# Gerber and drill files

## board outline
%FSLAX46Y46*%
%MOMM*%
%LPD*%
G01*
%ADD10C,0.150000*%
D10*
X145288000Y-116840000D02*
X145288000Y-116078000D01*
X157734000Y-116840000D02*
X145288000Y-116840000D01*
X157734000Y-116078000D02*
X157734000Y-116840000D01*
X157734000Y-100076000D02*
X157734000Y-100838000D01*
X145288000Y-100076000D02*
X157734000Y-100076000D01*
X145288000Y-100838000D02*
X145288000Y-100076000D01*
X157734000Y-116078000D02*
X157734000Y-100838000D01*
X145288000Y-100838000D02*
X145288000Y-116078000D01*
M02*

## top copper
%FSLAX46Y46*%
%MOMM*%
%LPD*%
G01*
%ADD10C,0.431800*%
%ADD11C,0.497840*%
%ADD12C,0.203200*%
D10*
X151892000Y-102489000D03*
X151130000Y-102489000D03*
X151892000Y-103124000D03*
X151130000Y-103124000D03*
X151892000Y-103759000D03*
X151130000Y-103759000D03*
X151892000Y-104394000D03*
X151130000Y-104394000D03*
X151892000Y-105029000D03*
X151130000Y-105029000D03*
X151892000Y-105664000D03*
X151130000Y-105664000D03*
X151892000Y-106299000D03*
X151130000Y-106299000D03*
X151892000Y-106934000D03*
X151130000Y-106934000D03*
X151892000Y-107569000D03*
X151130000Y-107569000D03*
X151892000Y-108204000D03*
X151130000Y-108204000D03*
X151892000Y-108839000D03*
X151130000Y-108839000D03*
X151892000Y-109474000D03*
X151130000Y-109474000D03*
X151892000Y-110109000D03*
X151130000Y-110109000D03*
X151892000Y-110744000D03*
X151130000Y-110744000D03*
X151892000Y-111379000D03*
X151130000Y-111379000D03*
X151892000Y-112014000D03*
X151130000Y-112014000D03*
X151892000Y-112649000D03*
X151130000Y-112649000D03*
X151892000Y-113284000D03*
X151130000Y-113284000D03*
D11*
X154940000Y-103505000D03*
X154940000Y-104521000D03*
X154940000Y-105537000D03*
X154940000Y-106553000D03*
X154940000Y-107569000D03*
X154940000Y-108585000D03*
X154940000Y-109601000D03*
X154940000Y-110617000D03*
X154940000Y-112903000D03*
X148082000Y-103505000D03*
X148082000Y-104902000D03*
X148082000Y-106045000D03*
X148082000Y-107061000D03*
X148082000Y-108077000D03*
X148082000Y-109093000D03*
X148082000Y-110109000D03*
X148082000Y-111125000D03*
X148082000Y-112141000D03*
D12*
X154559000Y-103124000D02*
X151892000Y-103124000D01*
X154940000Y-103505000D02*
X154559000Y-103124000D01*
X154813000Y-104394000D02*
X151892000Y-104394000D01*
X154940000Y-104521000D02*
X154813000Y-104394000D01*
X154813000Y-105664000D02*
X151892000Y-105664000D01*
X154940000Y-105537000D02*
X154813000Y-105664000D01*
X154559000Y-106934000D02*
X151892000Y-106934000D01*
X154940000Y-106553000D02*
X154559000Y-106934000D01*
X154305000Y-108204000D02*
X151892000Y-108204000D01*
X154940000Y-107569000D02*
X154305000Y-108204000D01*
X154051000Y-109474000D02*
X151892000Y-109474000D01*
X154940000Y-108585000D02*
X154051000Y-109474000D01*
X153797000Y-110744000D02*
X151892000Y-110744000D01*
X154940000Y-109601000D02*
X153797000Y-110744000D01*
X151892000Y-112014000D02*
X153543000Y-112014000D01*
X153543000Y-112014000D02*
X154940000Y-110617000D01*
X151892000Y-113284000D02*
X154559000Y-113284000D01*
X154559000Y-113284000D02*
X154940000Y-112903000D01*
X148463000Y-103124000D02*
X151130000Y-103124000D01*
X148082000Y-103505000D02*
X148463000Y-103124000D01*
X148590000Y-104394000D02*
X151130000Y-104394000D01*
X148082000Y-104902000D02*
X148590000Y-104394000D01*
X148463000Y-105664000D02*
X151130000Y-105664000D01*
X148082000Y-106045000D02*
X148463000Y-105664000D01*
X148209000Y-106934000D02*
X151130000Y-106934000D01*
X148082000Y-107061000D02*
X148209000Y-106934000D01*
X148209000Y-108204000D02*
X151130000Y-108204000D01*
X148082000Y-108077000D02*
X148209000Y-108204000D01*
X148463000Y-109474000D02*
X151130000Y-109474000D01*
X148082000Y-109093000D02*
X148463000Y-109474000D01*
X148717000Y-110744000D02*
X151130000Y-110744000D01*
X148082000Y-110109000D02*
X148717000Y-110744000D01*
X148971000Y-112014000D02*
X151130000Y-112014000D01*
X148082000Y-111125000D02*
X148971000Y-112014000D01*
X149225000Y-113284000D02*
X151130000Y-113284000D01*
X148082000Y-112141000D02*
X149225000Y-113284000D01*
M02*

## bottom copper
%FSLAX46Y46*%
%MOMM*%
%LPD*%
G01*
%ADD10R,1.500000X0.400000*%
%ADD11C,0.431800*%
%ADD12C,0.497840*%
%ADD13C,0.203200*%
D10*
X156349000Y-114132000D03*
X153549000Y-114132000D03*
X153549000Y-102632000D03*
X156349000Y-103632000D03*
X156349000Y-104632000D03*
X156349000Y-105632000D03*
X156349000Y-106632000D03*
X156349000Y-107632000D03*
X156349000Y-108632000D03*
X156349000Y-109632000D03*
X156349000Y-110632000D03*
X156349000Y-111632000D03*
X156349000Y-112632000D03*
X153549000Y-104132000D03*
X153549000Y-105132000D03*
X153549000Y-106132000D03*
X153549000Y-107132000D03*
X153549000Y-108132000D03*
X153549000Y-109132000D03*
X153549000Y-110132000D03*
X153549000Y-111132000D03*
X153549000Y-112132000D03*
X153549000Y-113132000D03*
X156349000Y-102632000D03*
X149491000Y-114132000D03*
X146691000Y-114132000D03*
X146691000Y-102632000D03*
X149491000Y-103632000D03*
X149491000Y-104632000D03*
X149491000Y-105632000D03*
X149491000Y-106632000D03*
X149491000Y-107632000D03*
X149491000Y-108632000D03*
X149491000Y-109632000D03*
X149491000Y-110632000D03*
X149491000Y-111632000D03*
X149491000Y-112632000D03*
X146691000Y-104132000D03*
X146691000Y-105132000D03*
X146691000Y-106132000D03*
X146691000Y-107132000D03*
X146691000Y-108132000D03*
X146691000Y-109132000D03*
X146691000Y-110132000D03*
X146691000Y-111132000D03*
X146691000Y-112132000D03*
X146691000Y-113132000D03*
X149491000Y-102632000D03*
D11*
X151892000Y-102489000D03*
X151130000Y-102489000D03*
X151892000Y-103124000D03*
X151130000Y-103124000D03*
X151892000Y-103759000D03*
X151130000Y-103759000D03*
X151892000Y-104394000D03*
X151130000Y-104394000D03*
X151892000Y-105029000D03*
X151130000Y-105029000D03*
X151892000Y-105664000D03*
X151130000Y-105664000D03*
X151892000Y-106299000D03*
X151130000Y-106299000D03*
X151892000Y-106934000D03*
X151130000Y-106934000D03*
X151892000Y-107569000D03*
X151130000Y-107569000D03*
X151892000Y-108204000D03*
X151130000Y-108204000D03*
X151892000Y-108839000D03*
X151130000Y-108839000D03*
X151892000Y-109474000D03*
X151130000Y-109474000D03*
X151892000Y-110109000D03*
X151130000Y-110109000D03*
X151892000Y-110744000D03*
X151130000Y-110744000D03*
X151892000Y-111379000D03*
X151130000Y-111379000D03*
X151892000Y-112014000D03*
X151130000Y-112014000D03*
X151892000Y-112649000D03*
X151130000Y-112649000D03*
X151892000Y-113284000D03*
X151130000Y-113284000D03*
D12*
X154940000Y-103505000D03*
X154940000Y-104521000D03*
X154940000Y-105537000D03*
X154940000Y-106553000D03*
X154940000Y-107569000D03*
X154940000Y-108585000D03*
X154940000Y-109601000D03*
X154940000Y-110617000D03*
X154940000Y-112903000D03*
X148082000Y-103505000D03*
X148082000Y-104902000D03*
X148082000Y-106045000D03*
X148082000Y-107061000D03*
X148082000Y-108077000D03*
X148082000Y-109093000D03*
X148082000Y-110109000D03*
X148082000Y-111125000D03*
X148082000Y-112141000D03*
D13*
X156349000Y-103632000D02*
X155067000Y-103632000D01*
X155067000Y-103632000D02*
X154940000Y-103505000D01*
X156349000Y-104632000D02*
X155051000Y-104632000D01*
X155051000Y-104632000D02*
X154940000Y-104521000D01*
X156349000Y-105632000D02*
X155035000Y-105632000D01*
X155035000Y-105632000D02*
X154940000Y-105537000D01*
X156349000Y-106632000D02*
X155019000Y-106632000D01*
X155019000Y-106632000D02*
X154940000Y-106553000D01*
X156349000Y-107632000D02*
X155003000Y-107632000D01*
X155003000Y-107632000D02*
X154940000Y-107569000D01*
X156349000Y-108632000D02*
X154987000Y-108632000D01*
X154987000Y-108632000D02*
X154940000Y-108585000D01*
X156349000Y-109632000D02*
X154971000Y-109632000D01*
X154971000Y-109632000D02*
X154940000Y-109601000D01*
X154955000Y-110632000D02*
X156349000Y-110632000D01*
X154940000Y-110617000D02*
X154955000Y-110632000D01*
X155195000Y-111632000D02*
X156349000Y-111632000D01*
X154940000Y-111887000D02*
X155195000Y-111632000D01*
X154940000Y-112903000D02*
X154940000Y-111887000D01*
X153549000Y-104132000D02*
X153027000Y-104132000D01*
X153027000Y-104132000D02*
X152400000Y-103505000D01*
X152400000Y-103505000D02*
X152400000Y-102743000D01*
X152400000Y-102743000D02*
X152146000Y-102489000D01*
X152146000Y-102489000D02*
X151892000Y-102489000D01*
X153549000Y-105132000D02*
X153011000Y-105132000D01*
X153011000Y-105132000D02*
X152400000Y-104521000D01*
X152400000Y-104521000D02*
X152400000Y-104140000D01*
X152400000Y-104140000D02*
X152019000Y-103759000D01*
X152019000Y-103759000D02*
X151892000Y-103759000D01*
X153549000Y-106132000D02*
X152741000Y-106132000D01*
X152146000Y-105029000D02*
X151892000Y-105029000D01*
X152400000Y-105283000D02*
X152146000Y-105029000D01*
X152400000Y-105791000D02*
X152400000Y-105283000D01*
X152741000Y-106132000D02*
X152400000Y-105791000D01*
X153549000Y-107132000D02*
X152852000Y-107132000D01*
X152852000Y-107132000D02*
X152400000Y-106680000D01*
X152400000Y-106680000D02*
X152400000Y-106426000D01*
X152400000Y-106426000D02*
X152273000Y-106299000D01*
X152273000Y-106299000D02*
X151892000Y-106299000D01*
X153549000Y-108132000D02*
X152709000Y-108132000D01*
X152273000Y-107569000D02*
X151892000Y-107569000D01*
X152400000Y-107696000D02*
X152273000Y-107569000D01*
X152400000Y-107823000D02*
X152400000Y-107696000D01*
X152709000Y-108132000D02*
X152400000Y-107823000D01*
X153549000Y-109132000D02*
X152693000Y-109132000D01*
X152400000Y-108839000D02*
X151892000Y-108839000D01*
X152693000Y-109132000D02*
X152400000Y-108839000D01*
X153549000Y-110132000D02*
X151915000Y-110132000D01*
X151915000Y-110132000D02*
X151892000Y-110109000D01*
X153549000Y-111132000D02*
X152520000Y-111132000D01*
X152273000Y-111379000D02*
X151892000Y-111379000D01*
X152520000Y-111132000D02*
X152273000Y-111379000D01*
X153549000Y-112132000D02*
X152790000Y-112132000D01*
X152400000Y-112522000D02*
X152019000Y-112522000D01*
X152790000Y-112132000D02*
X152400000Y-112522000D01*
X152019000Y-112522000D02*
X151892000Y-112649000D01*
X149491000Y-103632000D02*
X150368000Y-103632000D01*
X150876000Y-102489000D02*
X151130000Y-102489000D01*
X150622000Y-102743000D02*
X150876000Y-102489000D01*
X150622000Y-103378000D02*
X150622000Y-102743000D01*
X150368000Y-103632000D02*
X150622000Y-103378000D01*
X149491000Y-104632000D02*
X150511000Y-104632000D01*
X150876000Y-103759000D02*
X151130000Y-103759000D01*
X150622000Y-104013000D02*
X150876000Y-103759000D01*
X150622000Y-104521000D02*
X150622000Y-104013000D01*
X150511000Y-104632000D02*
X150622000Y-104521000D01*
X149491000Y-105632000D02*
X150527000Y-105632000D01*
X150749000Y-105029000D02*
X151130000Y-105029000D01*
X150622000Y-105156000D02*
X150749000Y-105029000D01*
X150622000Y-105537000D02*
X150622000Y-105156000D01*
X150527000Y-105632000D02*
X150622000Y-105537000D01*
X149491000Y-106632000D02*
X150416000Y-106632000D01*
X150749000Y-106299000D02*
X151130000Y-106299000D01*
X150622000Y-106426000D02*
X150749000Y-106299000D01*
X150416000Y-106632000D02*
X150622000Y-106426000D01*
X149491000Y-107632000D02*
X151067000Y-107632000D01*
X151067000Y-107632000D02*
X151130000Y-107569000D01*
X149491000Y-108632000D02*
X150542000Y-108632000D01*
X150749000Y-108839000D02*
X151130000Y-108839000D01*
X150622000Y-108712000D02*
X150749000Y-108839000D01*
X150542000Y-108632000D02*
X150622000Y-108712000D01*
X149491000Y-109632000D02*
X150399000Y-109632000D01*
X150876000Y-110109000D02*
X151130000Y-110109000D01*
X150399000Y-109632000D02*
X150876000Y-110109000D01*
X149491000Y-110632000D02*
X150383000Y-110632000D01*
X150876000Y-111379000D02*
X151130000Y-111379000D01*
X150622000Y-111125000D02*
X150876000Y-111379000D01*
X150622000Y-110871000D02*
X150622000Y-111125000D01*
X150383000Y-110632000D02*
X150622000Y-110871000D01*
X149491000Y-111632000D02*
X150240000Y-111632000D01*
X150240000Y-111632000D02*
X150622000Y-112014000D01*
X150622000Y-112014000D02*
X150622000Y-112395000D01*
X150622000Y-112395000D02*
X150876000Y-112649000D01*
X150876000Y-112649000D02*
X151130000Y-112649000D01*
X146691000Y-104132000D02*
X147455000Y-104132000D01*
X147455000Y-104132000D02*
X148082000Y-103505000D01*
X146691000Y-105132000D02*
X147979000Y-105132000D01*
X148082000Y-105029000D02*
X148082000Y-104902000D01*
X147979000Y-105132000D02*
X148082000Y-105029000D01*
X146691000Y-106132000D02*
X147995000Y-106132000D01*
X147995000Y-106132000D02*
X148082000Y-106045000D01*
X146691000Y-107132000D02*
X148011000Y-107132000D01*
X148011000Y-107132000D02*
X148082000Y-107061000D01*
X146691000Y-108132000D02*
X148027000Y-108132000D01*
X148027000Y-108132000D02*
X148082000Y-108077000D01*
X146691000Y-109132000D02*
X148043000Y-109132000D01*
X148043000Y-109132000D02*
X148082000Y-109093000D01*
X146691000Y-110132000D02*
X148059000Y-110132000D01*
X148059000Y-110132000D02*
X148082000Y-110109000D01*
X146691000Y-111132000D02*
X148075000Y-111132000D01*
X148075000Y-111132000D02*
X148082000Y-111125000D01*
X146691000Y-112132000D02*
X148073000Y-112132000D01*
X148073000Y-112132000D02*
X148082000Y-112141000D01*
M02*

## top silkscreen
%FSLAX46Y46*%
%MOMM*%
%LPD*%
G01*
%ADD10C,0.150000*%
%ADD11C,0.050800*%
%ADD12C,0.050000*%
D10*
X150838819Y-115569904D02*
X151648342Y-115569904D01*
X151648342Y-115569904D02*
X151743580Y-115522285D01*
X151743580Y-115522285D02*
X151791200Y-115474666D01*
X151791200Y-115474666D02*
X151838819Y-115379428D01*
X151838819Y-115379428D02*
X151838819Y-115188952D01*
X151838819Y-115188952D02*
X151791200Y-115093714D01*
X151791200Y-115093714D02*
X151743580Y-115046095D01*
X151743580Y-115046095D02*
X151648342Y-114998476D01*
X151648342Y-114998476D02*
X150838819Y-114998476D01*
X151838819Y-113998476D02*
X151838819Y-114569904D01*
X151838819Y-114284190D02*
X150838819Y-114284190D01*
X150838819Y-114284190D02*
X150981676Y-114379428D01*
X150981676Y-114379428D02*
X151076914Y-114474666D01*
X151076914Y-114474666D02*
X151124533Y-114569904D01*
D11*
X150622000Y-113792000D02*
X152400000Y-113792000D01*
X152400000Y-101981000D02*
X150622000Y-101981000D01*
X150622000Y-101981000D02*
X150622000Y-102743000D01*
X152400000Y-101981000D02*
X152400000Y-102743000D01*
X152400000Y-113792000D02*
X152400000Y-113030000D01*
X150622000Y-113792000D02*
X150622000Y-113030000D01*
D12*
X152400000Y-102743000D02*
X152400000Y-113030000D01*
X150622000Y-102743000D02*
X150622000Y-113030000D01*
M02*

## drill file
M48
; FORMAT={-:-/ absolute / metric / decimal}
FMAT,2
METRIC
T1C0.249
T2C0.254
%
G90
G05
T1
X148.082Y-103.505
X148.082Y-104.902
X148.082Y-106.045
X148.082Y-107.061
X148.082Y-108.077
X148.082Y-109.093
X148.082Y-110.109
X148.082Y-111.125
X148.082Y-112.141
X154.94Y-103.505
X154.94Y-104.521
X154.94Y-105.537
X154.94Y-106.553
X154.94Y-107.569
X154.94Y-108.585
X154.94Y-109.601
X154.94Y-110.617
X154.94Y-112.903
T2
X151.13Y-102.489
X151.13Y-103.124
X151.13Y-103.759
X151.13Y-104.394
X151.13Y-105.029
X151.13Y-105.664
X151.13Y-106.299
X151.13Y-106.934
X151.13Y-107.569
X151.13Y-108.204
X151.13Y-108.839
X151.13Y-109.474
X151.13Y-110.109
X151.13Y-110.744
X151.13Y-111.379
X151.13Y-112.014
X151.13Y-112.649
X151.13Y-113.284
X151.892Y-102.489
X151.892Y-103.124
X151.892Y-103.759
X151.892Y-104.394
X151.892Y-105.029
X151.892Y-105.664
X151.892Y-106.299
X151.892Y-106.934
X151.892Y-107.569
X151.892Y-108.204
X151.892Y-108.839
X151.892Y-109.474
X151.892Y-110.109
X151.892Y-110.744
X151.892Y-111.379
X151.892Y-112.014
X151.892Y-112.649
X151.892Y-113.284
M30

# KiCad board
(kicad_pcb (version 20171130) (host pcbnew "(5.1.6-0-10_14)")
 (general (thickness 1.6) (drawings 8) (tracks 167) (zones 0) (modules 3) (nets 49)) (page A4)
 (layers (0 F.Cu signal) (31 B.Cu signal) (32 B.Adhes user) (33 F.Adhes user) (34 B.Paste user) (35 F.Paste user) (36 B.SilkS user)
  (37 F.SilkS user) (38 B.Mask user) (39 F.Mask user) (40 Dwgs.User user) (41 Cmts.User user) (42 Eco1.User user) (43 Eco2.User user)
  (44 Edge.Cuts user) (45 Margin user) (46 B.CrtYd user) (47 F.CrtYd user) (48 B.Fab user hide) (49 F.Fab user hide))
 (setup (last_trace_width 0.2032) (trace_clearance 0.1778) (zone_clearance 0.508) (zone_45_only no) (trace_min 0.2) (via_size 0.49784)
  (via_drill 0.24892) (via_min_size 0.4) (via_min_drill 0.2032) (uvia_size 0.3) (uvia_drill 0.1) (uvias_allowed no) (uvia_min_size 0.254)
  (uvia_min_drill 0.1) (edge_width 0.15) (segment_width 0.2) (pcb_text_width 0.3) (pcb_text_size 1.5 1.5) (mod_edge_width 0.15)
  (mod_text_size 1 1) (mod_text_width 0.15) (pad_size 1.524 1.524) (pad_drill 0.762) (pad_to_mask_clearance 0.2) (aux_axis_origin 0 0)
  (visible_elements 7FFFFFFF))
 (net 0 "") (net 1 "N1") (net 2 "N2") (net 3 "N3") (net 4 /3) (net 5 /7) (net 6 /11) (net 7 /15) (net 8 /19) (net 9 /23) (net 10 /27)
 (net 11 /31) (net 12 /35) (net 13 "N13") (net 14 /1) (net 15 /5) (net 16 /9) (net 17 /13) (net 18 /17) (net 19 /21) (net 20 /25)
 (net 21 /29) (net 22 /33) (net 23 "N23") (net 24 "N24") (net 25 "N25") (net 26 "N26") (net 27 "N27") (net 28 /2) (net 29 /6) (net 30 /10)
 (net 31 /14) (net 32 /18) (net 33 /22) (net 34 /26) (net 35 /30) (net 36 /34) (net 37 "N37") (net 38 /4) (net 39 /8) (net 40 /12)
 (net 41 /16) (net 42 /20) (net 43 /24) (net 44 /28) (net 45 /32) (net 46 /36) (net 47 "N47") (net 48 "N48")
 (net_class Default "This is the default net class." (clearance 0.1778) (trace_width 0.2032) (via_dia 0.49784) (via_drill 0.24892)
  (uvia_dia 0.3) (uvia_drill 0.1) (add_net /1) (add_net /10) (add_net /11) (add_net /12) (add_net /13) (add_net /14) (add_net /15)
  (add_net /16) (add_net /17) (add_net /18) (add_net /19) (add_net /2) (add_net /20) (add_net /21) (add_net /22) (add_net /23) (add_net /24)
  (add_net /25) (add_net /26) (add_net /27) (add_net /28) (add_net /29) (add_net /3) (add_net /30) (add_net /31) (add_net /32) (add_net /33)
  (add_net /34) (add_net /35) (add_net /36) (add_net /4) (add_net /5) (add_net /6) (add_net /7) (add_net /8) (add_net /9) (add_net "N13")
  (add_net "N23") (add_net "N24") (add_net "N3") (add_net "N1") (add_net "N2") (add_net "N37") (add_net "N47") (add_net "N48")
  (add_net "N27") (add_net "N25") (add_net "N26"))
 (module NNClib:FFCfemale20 (layer B.Cu) (at 157.099 103.632 270)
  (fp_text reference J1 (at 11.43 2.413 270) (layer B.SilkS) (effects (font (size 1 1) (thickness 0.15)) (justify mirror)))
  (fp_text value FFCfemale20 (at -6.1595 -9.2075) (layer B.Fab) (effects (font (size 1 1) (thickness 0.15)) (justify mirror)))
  (pad 42 smd rect (at 10.5 0.75 270) (size 0.4 1.5) (layers B.Cu B.Paste B.Mask) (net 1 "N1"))
  (pad 43 smd rect (at 10.5 3.55 270) (size 0.4 1.5) (layers B.Cu B.Paste B.Mask) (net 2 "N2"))
  (pad 41 smd rect (at -1 3.55 270) (size 0.4 1.5) (layers B.Cu B.Paste B.Mask) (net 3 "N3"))
  (pad 1 smd rect (at 0 0.75 90) (size 0.4 1.5) (layers B.Cu B.Paste B.Mask) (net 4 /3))
  (pad 3 smd rect (at 1 0.75 90) (size 0.4 1.5) (layers B.Cu B.Paste B.Mask) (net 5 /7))
  (pad 5 smd rect (at 2 0.75 90) (size 0.4 1.5) (layers B.Cu B.Paste B.Mask) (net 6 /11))
  (pad 7 smd rect (at 3 0.75 90) (size 0.4 1.5) (layers B.Cu B.Paste B.Mask) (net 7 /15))
  (pad 9 smd rect (at 4 0.75 90) (size 0.4 1.5) (layers B.Cu B.Paste B.Mask) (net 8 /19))
  (pad 11 smd rect (at 5 0.75 90) (size 0.4 1.5) (layers B.Cu B.Paste B.Mask) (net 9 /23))
  (pad 13 smd rect (at 6 0.75 90) (size 0.4 1.5) (layers B.Cu B.Paste B.Mask) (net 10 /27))
  (pad 15 smd rect (at 7 0.75 90) (size 0.4 1.5) (layers B.Cu B.Paste B.Mask) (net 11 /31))
  (pad 17 smd rect (at 8 0.75 90) (size 0.4 1.5) (layers B.Cu B.Paste B.Mask) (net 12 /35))
  (pad 19 smd rect (at 9 0.75 90) (size 0.4 1.5) (layers B.Cu B.Paste B.Mask) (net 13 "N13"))
  (pad 2 smd rect (at 0.5 3.55 90) (size 0.4 1.5) (layers B.Cu B.Paste B.Mask) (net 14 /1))
  (pad 4 smd rect (at 1.5 3.55 90) (size 0.4 1.5) (layers B.Cu B.Paste B.Mask) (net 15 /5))
  (pad 6 smd rect (at 2.5 3.55 90) (size 0.4 1.5) (layers B.Cu B.Paste B.Mask) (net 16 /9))
  (pad 8 smd rect (at 3.5 3.55 90) (size 0.4 1.5) (layers B.Cu B.Paste B.Mask) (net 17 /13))
  (pad 10 smd rect (at 4.5 3.55 90) (size 0.4 1.5) (layers B.Cu B.Paste B.Mask) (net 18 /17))
  (pad 12 smd rect (at 5.5 3.55 90) (size 0.4 1.5) (layers B.Cu B.Paste B.Mask) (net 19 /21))
  (pad 14 smd rect (at 6.5 3.55 90) (size 0.4 1.5) (layers B.Cu B.Paste B.Mask) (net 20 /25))
  (pad 16 smd rect (at 7.5 3.55 90) (size 0.4 1.5) (layers B.Cu B.Paste B.Mask) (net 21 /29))
  (pad 18 smd rect (at 8.5 3.55 90) (size 0.4 1.5) (layers B.Cu B.Paste B.Mask) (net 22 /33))
  (pad 20 smd rect (at 9.5 3.55 90) (size 0.4 1.5) (layers B.Cu B.Paste B.Mask) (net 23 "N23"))
  (pad 40 smd rect (at -1 0.75 270) (size 0.4 1.5) (layers B.Cu B.Paste B.Mask) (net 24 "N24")))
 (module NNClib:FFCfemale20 (layer B.Cu) (at 150.241 103.632 270)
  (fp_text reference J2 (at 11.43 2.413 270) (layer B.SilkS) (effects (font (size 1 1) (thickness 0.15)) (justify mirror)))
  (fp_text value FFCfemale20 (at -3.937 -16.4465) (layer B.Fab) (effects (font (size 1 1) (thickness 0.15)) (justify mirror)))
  (pad 42 smd rect (at 10.5 0.75 270) (size 0.4 1.5) (layers B.Cu B.Paste B.Mask) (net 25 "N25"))
  (pad 43 smd rect (at 10.5 3.55 270) (size 0.4 1.5) (layers B.Cu B.Paste B.Mask) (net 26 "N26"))
  (pad 41 smd rect (at -1 3.55 270) (size 0.4 1.5) (layers B.Cu B.Paste B.Mask) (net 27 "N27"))
  (pad 1 smd rect (at 0 0.75 90) (size 0.4 1.5) (layers B.Cu B.Paste B.Mask) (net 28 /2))
  (pad 3 smd rect (at 1 0.75 90) (size 0.4 1.5) (layers B.Cu B.Paste B.Mask) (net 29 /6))
  (pad 5 smd rect (at 2 0.75 90) (size 0.4 1.5) (layers B.Cu B.Paste B.Mask) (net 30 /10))
  (pad 7 smd rect (at 3 0.75 90) (size 0.4 1.5) (layers B.Cu B.Paste B.Mask) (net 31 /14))
  (pad 9 smd rect (at 4 0.75 90) (size 0.4 1.5) (layers B.Cu B.Paste B.Mask) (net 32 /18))
  (pad 11 smd rect (at 5 0.75 90) (size 0.4 1.5) (layers B.Cu B.Paste B.Mask) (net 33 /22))
  (pad 13 smd rect (at 6 0.75 90) (size 0.4 1.5) (layers B.Cu B.Paste B.Mask) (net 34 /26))
  (pad 15 smd rect (at 7 0.75 90) (size 0.4 1.5) (layers B.Cu B.Paste B.Mask) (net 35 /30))
  (pad 17 smd rect (at 8 0.75 90) (size 0.4 1.5) (layers B.Cu B.Paste B.Mask) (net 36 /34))
  (pad 19 smd rect (at 9 0.75 90) (size 0.4 1.5) (layers B.Cu B.Paste B.Mask) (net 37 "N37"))
  (pad 2 smd rect (at 0.5 3.55 90) (size 0.4 1.5) (layers B.Cu B.Paste B.Mask) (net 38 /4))
  (pad 4 smd rect (at 1.5 3.55 90) (size 0.4 1.5) (layers B.Cu B.Paste B.Mask) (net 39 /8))
  (pad 6 smd rect (at 2.5 3.55 90) (size 0.4 1.5) (layers B.Cu B.Paste B.Mask) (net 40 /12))
  (pad 8 smd rect (at 3.5 3.55 90) (size 0.4 1.5) (layers B.Cu B.Paste B.Mask) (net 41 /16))
  (pad 10 smd rect (at 4.5 3.55 90) (size 0.4 1.5) (layers B.Cu B.Paste B.Mask) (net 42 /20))
  (pad 12 smd rect (at 5.5 3.55 90) (size 0.4 1.5) (layers B.Cu B.Paste B.Mask) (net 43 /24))
  (pad 14 smd rect (at 6.5 3.55 90) (size 0.4 1.5) (layers B.Cu B.Paste B.Mask) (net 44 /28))
  (pad 16 smd rect (at 7.5 3.55 90) (size 0.4 1.5) (layers B.Cu B.Paste B.Mask) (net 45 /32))
  (pad 18 smd rect (at 8.5 3.55 90) (size 0.4 1.5) (layers B.Cu B.Paste B.Mask) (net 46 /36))
  (pad 20 smd rect (at 9.5 3.55 90) (size 0.4 1.5) (layers B.Cu B.Paste B.Mask) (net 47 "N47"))
  (pad 40 smd rect (at -1 0.75 270) (size 0.4 1.5) (layers B.Cu B.Paste B.Mask) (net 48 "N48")))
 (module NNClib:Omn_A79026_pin (layer F.Cu) (at 150.114 102.489 270)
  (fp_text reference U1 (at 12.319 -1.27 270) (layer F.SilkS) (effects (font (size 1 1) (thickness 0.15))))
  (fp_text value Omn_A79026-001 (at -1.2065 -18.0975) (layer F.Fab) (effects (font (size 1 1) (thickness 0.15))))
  (fp_line (start 11.303 -0.508) (end 11.303 -2.286) (layer F.SilkS) (width 0.0508))
  (fp_line (start -0.508 -2.286) (end -0.508 -0.508) (layer F.SilkS) (width 0.0508))
  (fp_line (start -0.508 -0.508) (end 0.254 -0.508) (layer F.SilkS) (width 0.0508))
  (fp_line (start -0.508 -2.286) (end 0.254 -2.286) (layer F.SilkS) (width 0.0508))
  (fp_line (start 11.303 -2.286) (end 10.541 -2.286) (layer F.SilkS) (width 0.0508))
  (fp_line (start 11.303 -0.508) (end 10.541 -0.508) (layer F.SilkS) (width 0.0508))
  (fp_line (start 0.254 -2.286) (end 10.541 -2.286) (layer F.SilkS) (width 0.05))
  (fp_line (start 0.254 -0.508) (end 10.541 -0.508) (layer F.SilkS) (width 0.05))
  (pad 1 thru_hole circle (at 0 -1.778 270) (size 0.4318 0.4318) (drill 0.254) (layers *.Cu *.Mask) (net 14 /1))
  (pad 2 thru_hole circle (at 0 -1.016 270) (size 0.4318 0.4318) (drill 0.254) (layers *.Cu *.Mask) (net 28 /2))
  (pad 3 thru_hole circle (at 0.635 -1.778 270) (size 0.4318 0.4318) (drill 0.254) (layers *.Cu *.Mask) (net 4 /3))
  (pad 4 thru_hole circle (at 0.635 -1.016 270) (size 0.4318 0.4318) (drill 0.254) (layers *.Cu *.Mask) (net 38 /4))
  (pad 5 thru_hole circle (at 1.27 -1.778 270) (size 0.4318 0.4318) (drill 0.254) (layers *.Cu *.Mask) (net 15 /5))
  (pad 6 thru_hole circle (at 1.27 -1.016 270) (size 0.4318 0.4318) (drill 0.254) (layers *.Cu *.Mask) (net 29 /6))
  (pad 7 thru_hole circle (at 1.905 -1.778 270) (size 0.4318 0.4318) (drill 0.254) (layers *.Cu *.Mask) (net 5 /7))
  (pad 8 thru_hole circle (at 1.905 -1.016 270) (size 0.4318 0.4318) (drill 0.254) (layers *.Cu *.Mask) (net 39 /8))
  (pad 9 thru_hole circle (at 2.54 -1.778 270) (size 0.4318 0.4318) (drill 0.254) (layers *.Cu *.Mask) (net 16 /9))
  (pad 10 thru_hole circle (at 2.54 -1.016 270) (size 0.4318 0.4318) (drill 0.254) (layers *.Cu *.Mask) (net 30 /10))
  (pad 11 thru_hole circle (at 3.175 -1.778 270) (size 0.4318 0.4318) (drill 0.254) (layers *.Cu *.Mask) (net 6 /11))
  (pad 12 thru_hole circle (at 3.175 -1.016 270) (size 0.4318 0.4318) (drill 0.254) (layers *.Cu *.Mask) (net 40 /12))
  (pad 13 thru_hole circle (at 3.81 -1.778 270) (size 0.4318 0.4318) (drill 0.254) (layers *.Cu *.Mask) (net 17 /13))
  (pad 14 thru_hole circle (at 3.81 -1.016 270) (size 0.4318 0.4318) (drill 0.254) (layers *.Cu *.Mask) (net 31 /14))
  (pad 15 thru_hole circle (at 4.445 -1.778 270) (size 0.4318 0.4318) (drill 0.254) (layers *.Cu *.Mask) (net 7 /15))
  (pad 16 thru_hole circle (at 4.445 -1.016 270) (size 0.4318 0.4318) (drill 0.254) (layers *.Cu *.Mask) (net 41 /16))
  (pad 17 thru_hole circle (at 5.08 -1.778 270) (size 0.4318 0.4318) (drill 0.254) (layers *.Cu *.Mask) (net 18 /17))
  (pad 18 thru_hole circle (at 5.08 -1.016 270) (size 0.4318 0.4318) (drill 0.254) (layers *.Cu *.Mask) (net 32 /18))
  (pad 19 thru_hole circle (at 5.715 -1.778 270) (size 0.4318 0.4318) (drill 0.254) (layers *.Cu *.Mask) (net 8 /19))
  (pad 20 thru_hole circle (at 5.715 -1.016 270) (size 0.4318 0.4318) (drill 0.254) (layers *.Cu *.Mask) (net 42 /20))
  (pad 21 thru_hole circle (at 6.35 -1.778 270) (size 0.4318 0.4318) (drill 0.254) (layers *.Cu *.Mask) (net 19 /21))
  (pad 22 thru_hole circle (at 6.35 -1.016 270) (size 0.4318 0.4318) (drill 0.254) (layers *.Cu *.Mask) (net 33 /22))
  (pad 23 thru_hole circle (at 6.985 -1.778 270) (size 0.4318 0.4318) (drill 0.254) (layers *.Cu *.Mask) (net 9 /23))
  (pad 24 thru_hole circle (at 6.985 -1.016 270) (size 0.4318 0.4318) (drill 0.254) (layers *.Cu *.Mask) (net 43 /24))
  (pad 25 thru_hole circle (at 7.62 -1.778 270) (size 0.4318 0.4318) (drill 0.254) (layers *.Cu *.Mask) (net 20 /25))
  (pad 26 thru_hole circle (at 7.62 -1.016 270) (size 0.4318 0.4318) (drill 0.254) (layers *.Cu *.Mask) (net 34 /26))
  (pad 27 thru_hole circle (at 8.255 -1.778 270) (size 0.4318 0.4318) (drill 0.254) (layers *.Cu *.Mask) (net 10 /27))
  (pad 28 thru_hole circle (at 8.255 -1.016 270) (size 0.4318 0.4318) (drill 0.254) (layers *.Cu *.Mask) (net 44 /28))
  (pad 29 thru_hole circle (at 8.89 -1.778 270) (size 0.4318 0.4318) (drill 0.254) (layers *.Cu *.Mask) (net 21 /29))
  (pad 30 thru_hole circle (at 8.89 -1.016 270) (size 0.4318 0.4318) (drill 0.254) (layers *.Cu *.Mask) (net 35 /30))
  (pad 31 thru_hole circle (at 9.525 -1.778 270) (size 0.4318 0.4318) (drill 0.254) (layers *.Cu *.Mask) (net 11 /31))
  (pad 32 thru_hole circle (at 9.525 -1.016 270) (size 0.4318 0.4318) (drill 0.254) (layers *.Cu *.Mask) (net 45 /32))
  (pad 33 thru_hole circle (at 10.16 -1.778 270) (size 0.4318 0.4318) (drill 0.254) (layers *.Cu *.Mask) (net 22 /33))
  (pad 34 thru_hole circle (at 10.16 -1.016 270) (size 0.4318 0.4318) (drill 0.254) (layers *.Cu *.Mask) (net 36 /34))
  (pad 35 thru_hole circle (at 10.795 -1.778 270) (size 0.4318 0.4318) (drill 0.254) (layers *.Cu *.Mask) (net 12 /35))
  (pad 36 thru_hole circle (at 10.795 -1.016 270) (size 0.4318 0.4318) (drill 0.254) (layers *.Cu *.Mask) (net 46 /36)))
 (gr_line (start 145.288 116.84) (end 145.288 116.078) (angle 90) (layer Edge.Cuts) (width 0.15))
 (gr_line (start 157.734 116.84) (end 145.288 116.84) (angle 90) (layer Edge.Cuts) (width 0.15))
 (gr_line (start 157.734 116.078) (end 157.734 116.84) (angle 90) (layer Edge.Cuts) (width 0.15))
 (gr_line (start 157.734 100.076) (end 157.734 100.838) (angle 90) (layer Edge.Cuts) (width 0.15))
 (gr_line (start 145.288 100.076) (end 157.734 100.076) (angle 90) (layer Edge.Cuts) (width 0.15))
 (gr_line (start 145.288 100.838) (end 145.288 100.076) (angle 90) (layer Edge.Cuts) (width 0.15))
 (gr_line (start 157.734 116.078) (end 157.734 100.838) (angle 90) (layer Edge.Cuts) (width 0.15))
 (gr_line (start 145.288 100.838) (end 145.288 116.078) (angle 90) (layer Edge.Cuts) (width 0.15))
 (segment (start 156.349 103.632) (end 155.067 103.632) (width 0.2032) (layer B.Cu) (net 4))
 (segment (start 154.559 103.124) (end 151.892 103.124) (width 0.2032) (layer F.Cu) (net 4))
 (segment (start 154.94 103.505) (end 154.559 103.124) (width 0.2032) (layer F.Cu) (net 4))
 (via (at 154.94 103.505) (size 0.49784) (drill 0.24892) (layers F.Cu B.Cu) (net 4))
 (segment (start 155.067 103.632) (end 154.94 103.505) (width 0.2032) (layer B.Cu) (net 4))
 (segment (start 156.349 104.632) (end 155.051 104.632) (width 0.2032) (layer B.Cu) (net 5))
 (segment (start 154.813 104.394) (end 151.892 104.394) (width 0.2032) (layer F.Cu) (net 5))
 (segment (start 154.94 104.521) (end 154.813 104.394) (width 0.2032) (layer F.Cu) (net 5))
 (via (at 154.94 104.521) (size 0.49784) (drill 0.24892) (layers F.Cu B.Cu) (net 5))
 (segment (start 155.051 104.632) (end 154.94 104.521) (width 0.2032) (layer B.Cu) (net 5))
 (segment (start 156.349 105.632) (end 155.035 105.632) (width 0.2032) (layer B.Cu) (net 6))
 (segment (start 154.813 105.664) (end 151.892 105.664) (width 0.2032) (layer F.Cu) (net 6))
 (segment (start 154.94 105.537) (end 154.813 105.664) (width 0.2032) (layer F.Cu) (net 6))
 (via (at 154.94 105.537) (size 0.49784) (drill 0.24892) (layers F.Cu B.Cu) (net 6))
 (segment (start 155.035 105.632) (end 154.94 105.537) (width 0.2032) (layer B.Cu) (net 6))
 (segment (start 156.349 106.632) (end 155.019 106.632) (width 0.2032) (layer B.Cu) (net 7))
 (segment (start 154.559 106.934) (end 151.892 106.934) (width 0.2032) (layer F.Cu) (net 7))
 (segment (start 154.94 106.553) (end 154.559 106.934) (width 0.2032) (layer F.Cu) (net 7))
 (via (at 154.94 106.553) (size 0.49784) (drill 0.24892) (layers F.Cu B.Cu) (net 7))
 (segment (start 155.019 106.632) (end 154.94 106.553) (width 0.2032) (layer B.Cu) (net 7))
 (segment (start 156.349 107.632) (end 155.003 107.632) (width 0.2032) (layer B.Cu) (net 8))
 (segment (start 154.305 108.204) (end 151.892 108.204) (width 0.2032) (layer F.Cu) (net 8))
 (segment (start 154.94 107.569) (end 154.305 108.204) (width 0.2032) (layer F.Cu) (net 8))
 (via (at 154.94 107.569) (size 0.49784) (drill 0.24892) (layers F.Cu B.Cu) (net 8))
 (segment (start 155.003 107.632) (end 154.94 107.569) (width 0.2032) (layer B.Cu) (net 8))
 (segment (start 156.349 108.632) (end 154.987 108.632) (width 0.2032) (layer B.Cu) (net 9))
 (segment (start 154.051 109.474) (end 151.892 109.474) (width 0.2032) (layer F.Cu) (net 9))
 (segment (start 154.94 108.585) (end 154.051 109.474) (width 0.2032) (layer F.Cu) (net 9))
 (via (at 154.94 108.585) (size 0.49784) (drill 0.24892) (layers F.Cu B.Cu) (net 9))
 (segment (start 154.987 108.632) (end 154.94 108.585) (width 0.2032) (layer B.Cu) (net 9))
 (segment (start 156.349 109.632) (end 154.971 109.632) (width 0.2032) (layer B.Cu) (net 10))
 (segment (start 153.797 110.744) (end 151.892 110.744) (width 0.2032) (layer F.Cu) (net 10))
 (segment (start 154.94 109.601) (end 153.797 110.744) (width 0.2032) (layer F.Cu) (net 10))
 (via (at 154.94 109.601) (size 0.49784) (drill 0.24892) (layers F.Cu B.Cu) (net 10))
 (segment (start 154.971 109.632) (end 154.94 109.601) (width 0.2032) (layer B.Cu) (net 10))
 (segment (start 151.892 112.014) (end 153.543 112.014) (width 0.2032) (layer F.Cu) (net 11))
 (segment (start 154.955 110.632) (end 156.349 110.632) (width 0.2032) (layer B.Cu) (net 11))
 (segment (start 154.94 110.617) (end 154.955 110.632) (width 0.2032) (layer B.Cu) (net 11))
 (via (at 154.94 110.617) (size 0.49784) (drill 0.24892) (layers F.Cu B.Cu) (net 11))
 (segment (start 153.543 112.014) (end 154.94 110.617) (width 0.2032) (layer F.Cu) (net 11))
 (segment (start 151.892 113.284) (end 154.559 113.284) (width 0.2032) (layer F.Cu) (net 12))
 (segment (start 155.195 111.632) (end 156.349 111.632) (width 0.2032) (layer B.Cu) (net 12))
 (segment (start 154.94 111.887) (end 155.195 111.632) (width 0.2032) (layer B.Cu) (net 12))
 (segment (start 154.94 112.903) (end 154.94 111.887) (width 0.2032) (layer B.Cu) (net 12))
 (via (at 154.94 112.903) (size 0.49784) (drill 0.24892) (layers F.Cu B.Cu) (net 12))
 (segment (start 154.559 113.284) (end 154.94 112.903) (width 0.2032) (layer F.Cu) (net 12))
 (segment (start 153.549 104.132) (end 153.027 104.132) (width 0.2032) (layer B.Cu) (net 14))
 (segment (start 153.027 104.132) (end 152.4 103.505) (width 0.2032) (layer B.Cu) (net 14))
 (segment (start 152.4 103.505) (end 152.4 102.743) (width 0.2032) (layer B.Cu) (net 14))
 (segment (start 152.4 102.743) (end 152.146 102.489) (width 0.2032) (layer B.Cu) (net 14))
 (segment (start 152.146 102.489) (end 151.892 102.489) (width 0.2032) (layer B.Cu) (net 14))
 (segment (start 153.549 105.132) (end 153.011 105.132) (width 0.2032) (layer B.Cu) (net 15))
 (segment (start 153.011 105.132) (end 152.4 104.521) (width 0.2032) (layer B.Cu) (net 15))
 (segment (start 152.4 104.521) (end 152.4 104.14) (width 0.2032) (layer B.Cu) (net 15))
 (segment (start 152.4 104.14) (end 152.019 103.759) (width 0.2032) (layer B.Cu) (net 15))
 (segment (start 152.019 103.759) (end 151.892 103.759) (width 0.2032) (layer B.Cu) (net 15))
 (segment (start 153.549 106.132) (end 152.741 106.132) (width 0.2032) (layer B.Cu) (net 16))
 (segment (start 152.146 105.029) (end 151.892 105.029) (width 0.2032) (layer B.Cu) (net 16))
 (segment (start 152.4 105.283) (end 152.146 105.029) (width 0.2032) (layer B.Cu) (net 16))
 (segment (start 152.4 105.791) (end 152.4 105.283) (width 0.2032) (layer B.Cu) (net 16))
 (segment (start 152.741 106.132) (end 152.4 105.791) (width 0.2032) (layer B.Cu) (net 16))
 (segment (start 153.549 107.132) (end 152.852 107.132) (width 0.2032) (layer B.Cu) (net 17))
 (segment (start 152.852 107.132) (end 152.4 106.68) (width 0.2032) (layer B.Cu) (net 17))
 (segment (start 152.4 106.68) (end 152.4 106.426) (width 0.2032) (layer B.Cu) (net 17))
 (segment (start 152.4 106.426) (end 152.273 106.299) (width 0.2032) (layer B.Cu) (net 17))
 (segment (start 152.273 106.299) (end 151.892 106.299) (width 0.2032) (layer B.Cu) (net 17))
 (segment (start 153.549 108.132) (end 152.709 108.132) (width 0.2032) (layer B.Cu) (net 18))
 (segment (start 152.273 107.569) (end 151.892 107.569) (width 0.2032) (layer B.Cu) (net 18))
 (segment (start 152.4 107.696) (end 152.273 107.569) (width 0.2032) (layer B.Cu) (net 18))
 (segment (start 152.4 107.823) (end 152.4 107.696) (width 0.2032) (layer B.Cu) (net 18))
 (segment (start 152.709 108.132) (end 152.4 107.823) (width 0.2032) (layer B.Cu) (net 18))
 (segment (start 153.549 109.132) (end 152.693 109.132) (width 0.2032) (layer B.Cu) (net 19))
 (segment (start 152.4 108.839) (end 151.892 108.839) (width 0.2032) (layer B.Cu) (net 19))
 (segment (start 152.693 109.132) (end 152.4 108.839) (width 0.2032) (layer B.Cu) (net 19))
 (segment (start 153.549 110.132) (end 151.915 110.132) (width 0.2032) (layer B.Cu) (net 20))
 (segment (start 151.915 110.132) (end 151.892 110.109) (width 0.2032) (layer B.Cu) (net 20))
 (segment (start 153.549 111.132) (end 152.52 111.132) (width 0.2032) (layer B.Cu) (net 21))
 (segment (start 152.273 111.379) (end 151.892 111.379) (width 0.2032) (layer B.Cu) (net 21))
 (segment (start 152.52 111.132) (end 152.273 111.379) (width 0.2032) (layer B.Cu) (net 21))
 (segment (start 153.549 112.132) (end 152.79 112.132) (width 0.2032) (layer B.Cu) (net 22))
 (segment (start 152.4 112.522) (end 152.019 112.522) (width 0.2032) (layer B.Cu) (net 22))
 (segment (start 152.79 112.132) (end 152.4 112.522) (width 0.2032) (layer B.Cu) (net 22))
 (segment (start 152.019 112.522) (end 151.892 112.649) (width 0.2032) (layer B.Cu) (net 22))
 (segment (start 149.491 103.632) (end 150.368 103.632) (width 0.2032) (layer B.Cu) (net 28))
 (segment (start 150.876 102.489) (end 151.13 102.489) (width 0.2032) (layer B.Cu) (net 28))
 (segment (start 150.622 102.743) (end 150.876 102.489) (width 0.2032) (layer B.Cu) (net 28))
 (segment (start 150.622 103.378) (end 150.622 102.743) (width 0.2032) (layer B.Cu) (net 28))
 (segment (start 150.368 103.632) (end 150.622 103.378) (width 0.2032) (layer B.Cu) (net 28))
 (segment (start 149.491 104.632) (end 150.511 104.632) (width 0.2032) (layer B.Cu) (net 29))
 (segment (start 150.876 103.759) (end 151.13 103.759) (width 0.2032) (layer B.Cu) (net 29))
 (segment (start 150.622 104.013) (end 150.876 103.759) (width 0.2032) (layer B.Cu) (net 29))
 (segment (start 150.622 104.521) (end 150.622 104.013) (width 0.2032) (layer B.Cu) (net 29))
 (segment (start 150.511 104.632) (end 150.622 104.521) (width 0.2032) (layer B.Cu) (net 29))
 (segment (start 149.491 105.632) (end 150.527 105.632) (width 0.2032) (layer B.Cu) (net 30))
 (segment (start 150.749 105.029) (end 151.13 105.029) (width 0.2032) (layer B.Cu) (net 30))
 (segment (start 150.622 105.156) (end 150.749 105.029) (width 0.2032) (layer B.Cu) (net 30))
 (segment (start 150.622 105.537) (end 150.622 105.156) (width 0.2032) (layer B.Cu) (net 30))
 (segment (start 150.527 105.632) (end 150.622 105.537) (width 0.2032) (layer B.Cu) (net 30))
 (segment (start 149.491 106.632) (end 150.416 106.632) (width 0.2032) (layer B.Cu) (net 31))
 (segment (start 150.749 106.299) (end 151.13 106.299) (width 0.2032) (layer B.Cu) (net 31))
 (segment (start 150.622 106.426) (end 150.749 106.299) (width 0.2032) (layer B.Cu) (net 31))
 (segment (start 150.416 106.632) (end 150.622 106.426) (width 0.2032) (layer B.Cu) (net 31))
 (segment (start 149.491 107.632) (end 151.067 107.632) (width 0.2032) (layer B.Cu) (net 32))
 (segment (start 151.067 107.632) (end 151.13 107.569) (width 0.2032) (layer B.Cu) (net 32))
 (segment (start 149.491 108.632) (end 150.542 108.632) (width 0.2032) (layer B.Cu) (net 33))
 (segment (start 150.749 108.839) (end 151.13 108.839) (width 0.2032) (layer B.Cu) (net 33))
 (segment (start 150.622 108.712) (end 150.749 108.839) (width 0.2032) (layer B.Cu) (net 33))
 (segment (start 150.542 108.632) (end 150.622 108.712) (width 0.2032) (layer B.Cu) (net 33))
 (segment (start 149.491 109.632) (end 150.399 109.632) (width 0.2032) (layer B.Cu) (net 34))
 (segment (start 150.876 110.109) (end 151.13 110.109) (width 0.2032) (layer B.Cu) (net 34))
 (segment (start 150.399 109.632) (end 150.876 110.109) (width 0.2032) (layer B.Cu) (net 34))
 (segment (start 149.491 110.632) (end 150.383 110.632) (width 0.2032) (layer B.Cu) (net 35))
 (segment (start 150.876 111.379) (end 151.13 111.379) (width 0.2032) (layer B.Cu) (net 35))
 (segment (start 150.622 111.125) (end 150.876 111.379) (width 0.2032) (layer B.Cu) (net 35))
 (segment (start 150.622 110.871) (end 150.622 111.125) (width 0.2032) (layer B.Cu) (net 35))
 (segment (start 150.383 110.632) (end 150.622 110.871) (width 0.2032) (layer B.Cu) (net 35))
 (segment (start 149.491 111.632) (end 150.24 111.632) (width 0.2032) (layer B.Cu) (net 36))
 (segment (start 150.24 111.632) (end 150.622 112.014) (width 0.2032) (layer B.Cu) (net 36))
 (segment (start 150.622 112.014) (end 150.622 112.395) (width 0.2032) (layer B.Cu) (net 36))
 (segment (start 150.622 112.395) (end 150.876 112.649) (width 0.2032) (layer B.Cu) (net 36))
 (segment (start 150.876 112.649) (end 151.13 112.649) (width 0.2032) (layer B.Cu) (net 36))
 (segment (start 146.691 104.132) (end 147.455 104.132) (width 0.2032) (layer B.Cu) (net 38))
 (segment (start 148.463 103.124) (end 151.13 103.124) (width 0.2032) (layer F.Cu) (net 38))
 (segment (start 148.082 103.505) (end 148.463 103.124) (width 0.2032) (layer F.Cu) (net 38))
 (via (at 148.082 103.505) (size 0.49784) (drill 0.24892) (layers F.Cu B.Cu) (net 38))
 (segment (start 147.455 104.132) (end 148.082 103.505) (width 0.2032) (layer B.Cu) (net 38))
 (segment (start 146.691 105.132) (end 147.979 105.132) (width 0.2032) (layer B.Cu) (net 39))
 (segment (start 148.59 104.394) (end 151.13 104.394) (width 0.2032) (layer F.Cu) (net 39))
 (segment (start 148.082 104.902) (end 148.59 104.394) (width 0.2032) (layer F.Cu) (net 39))
 (via (at 148.082 104.902) (size 0.49784) (drill 0.24892) (layers F.Cu B.Cu) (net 39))
 (segment (start 148.082 105.029) (end 148.082 104.902) (width 0.2032) (layer B.Cu) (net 39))
 (segment (start 147.979 105.132) (end 148.082 105.029) (width 0.2032) (layer B.Cu) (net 39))
 (segment (start 146.691 106.132) (end 147.995 106.132) (width 0.2032) (layer B.Cu) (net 40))
 (segment (start 148.463 105.664) (end 151.13 105.664) (width 0.2032) (layer F.Cu) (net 40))
 (segment (start 148.082 106.045) (end 148.463 105.664) (width 0.2032) (layer F.Cu) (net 40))
 (via (at 148.082 106.045) (size 0.49784) (drill 0.24892) (layers F.Cu B.Cu) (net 40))
 (segment (start 147.995 106.132) (end 148.082 106.045) (width 0.2032) (layer B.Cu) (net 40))
 (segment (start 146.691 107.132) (end 148.011 107.132) (width 0.2032) (layer B.Cu) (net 41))
 (segment (start 148.209 106.934) (end 151.13 106.934) (width 0.2032) (layer F.Cu) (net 41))
 (segment (start 148.082 107.061) (end 148.209 106.934) (width 0.2032) (layer F.Cu) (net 41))
 (via (at 148.082 107.061) (size 0.49784) (drill 0.24892) (layers F.Cu B.Cu) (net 41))
 (segment (start 148.011 107.132) (end 148.082 107.061) (width 0.2032) (layer B.Cu) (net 41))
 (segment (start 146.691 108.132) (end 148.027 108.132) (width 0.2032) (layer B.Cu) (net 42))
 (segment (start 148.209 108.204) (end 151.13 108.204) (width 0.2032) (layer F.Cu) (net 42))
 (segment (start 148.082 108.077) (end 148.209 108.204) (width 0.2032) (layer F.Cu) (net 42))
 (via (at 148.082 108.077) (size 0.49784) (drill 0.24892) (layers F.Cu B.Cu) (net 42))
 (segment (start 148.027 108.132) (end 148.082 108.077) (width 0.2032) (layer B.Cu) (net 42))
 (segment (start 146.691 109.132) (end 148.043 109.132) (width 0.2032) (layer B.Cu) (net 43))
 (segment (start 148.463 109.474) (end 151.13 109.474) (width 0.2032) (layer F.Cu) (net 43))
 (segment (start 148.082 109.093) (end 148.463 109.474) (width 0.2032) (layer F.Cu) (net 43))
 (via (at 148.082 109.093) (size 0.49784) (drill 0.24892) (layers F.Cu B.Cu) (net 43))
 (segment (start 148.043 109.132) (end 148.082 109.093) (width 0.2032) (layer B.Cu) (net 43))
 (segment (start 146.691 110.132) (end 148.059 110.132) (width 0.2032) (layer B.Cu) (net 44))
 (segment (start 148.717 110.744) (end 151.13 110.744) (width 0.2032) (layer F.Cu) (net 44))
 (segment (start 148.082 110.109) (end 148.717 110.744) (width 0.2032) (layer F.Cu) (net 44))
 (via (at 148.082 110.109) (size 0.49784) (drill 0.24892) (layers F.Cu B.Cu) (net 44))
 (segment (start 148.059 110.132) (end 148.082 110.109) (width 0.2032) (layer B.Cu) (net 44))
 (segment (start 146.691 111.132) (end 148.075 111.132) (width 0.2032) (layer B.Cu) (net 45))
 (segment (start 148.971 112.014) (end 151.13 112.014) (width 0.2032) (layer F.Cu) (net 45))
 (segment (start 148.082 111.125) (end 148.971 112.014) (width 0.2032) (layer F.Cu) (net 45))
 (via (at 148.082 111.125) (size 0.49784) (drill 0.24892) (layers F.Cu B.Cu) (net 45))
 (segment (start 148.075 111.132) (end 148.082 111.125) (width 0.2032) (layer B.Cu) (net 45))
 (segment (start 146.691 112.132) (end 148.073 112.132) (width 0.2032) (layer B.Cu) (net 46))
 (segment (start 149.225 113.284) (end 151.13 113.284) (width 0.2032) (layer F.Cu) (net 46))
 (segment (start 148.082 112.141) (end 149.225 113.284) (width 0.2032) (layer F.Cu) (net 46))
 (via (at 148.082 112.141) (size 0.49784) (drill 0.24892) (layers F.Cu B.Cu) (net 46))
 (segment (start 148.073 112.132) (end 148.082 112.141) (width 0.2032) (layer B.Cu) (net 46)))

